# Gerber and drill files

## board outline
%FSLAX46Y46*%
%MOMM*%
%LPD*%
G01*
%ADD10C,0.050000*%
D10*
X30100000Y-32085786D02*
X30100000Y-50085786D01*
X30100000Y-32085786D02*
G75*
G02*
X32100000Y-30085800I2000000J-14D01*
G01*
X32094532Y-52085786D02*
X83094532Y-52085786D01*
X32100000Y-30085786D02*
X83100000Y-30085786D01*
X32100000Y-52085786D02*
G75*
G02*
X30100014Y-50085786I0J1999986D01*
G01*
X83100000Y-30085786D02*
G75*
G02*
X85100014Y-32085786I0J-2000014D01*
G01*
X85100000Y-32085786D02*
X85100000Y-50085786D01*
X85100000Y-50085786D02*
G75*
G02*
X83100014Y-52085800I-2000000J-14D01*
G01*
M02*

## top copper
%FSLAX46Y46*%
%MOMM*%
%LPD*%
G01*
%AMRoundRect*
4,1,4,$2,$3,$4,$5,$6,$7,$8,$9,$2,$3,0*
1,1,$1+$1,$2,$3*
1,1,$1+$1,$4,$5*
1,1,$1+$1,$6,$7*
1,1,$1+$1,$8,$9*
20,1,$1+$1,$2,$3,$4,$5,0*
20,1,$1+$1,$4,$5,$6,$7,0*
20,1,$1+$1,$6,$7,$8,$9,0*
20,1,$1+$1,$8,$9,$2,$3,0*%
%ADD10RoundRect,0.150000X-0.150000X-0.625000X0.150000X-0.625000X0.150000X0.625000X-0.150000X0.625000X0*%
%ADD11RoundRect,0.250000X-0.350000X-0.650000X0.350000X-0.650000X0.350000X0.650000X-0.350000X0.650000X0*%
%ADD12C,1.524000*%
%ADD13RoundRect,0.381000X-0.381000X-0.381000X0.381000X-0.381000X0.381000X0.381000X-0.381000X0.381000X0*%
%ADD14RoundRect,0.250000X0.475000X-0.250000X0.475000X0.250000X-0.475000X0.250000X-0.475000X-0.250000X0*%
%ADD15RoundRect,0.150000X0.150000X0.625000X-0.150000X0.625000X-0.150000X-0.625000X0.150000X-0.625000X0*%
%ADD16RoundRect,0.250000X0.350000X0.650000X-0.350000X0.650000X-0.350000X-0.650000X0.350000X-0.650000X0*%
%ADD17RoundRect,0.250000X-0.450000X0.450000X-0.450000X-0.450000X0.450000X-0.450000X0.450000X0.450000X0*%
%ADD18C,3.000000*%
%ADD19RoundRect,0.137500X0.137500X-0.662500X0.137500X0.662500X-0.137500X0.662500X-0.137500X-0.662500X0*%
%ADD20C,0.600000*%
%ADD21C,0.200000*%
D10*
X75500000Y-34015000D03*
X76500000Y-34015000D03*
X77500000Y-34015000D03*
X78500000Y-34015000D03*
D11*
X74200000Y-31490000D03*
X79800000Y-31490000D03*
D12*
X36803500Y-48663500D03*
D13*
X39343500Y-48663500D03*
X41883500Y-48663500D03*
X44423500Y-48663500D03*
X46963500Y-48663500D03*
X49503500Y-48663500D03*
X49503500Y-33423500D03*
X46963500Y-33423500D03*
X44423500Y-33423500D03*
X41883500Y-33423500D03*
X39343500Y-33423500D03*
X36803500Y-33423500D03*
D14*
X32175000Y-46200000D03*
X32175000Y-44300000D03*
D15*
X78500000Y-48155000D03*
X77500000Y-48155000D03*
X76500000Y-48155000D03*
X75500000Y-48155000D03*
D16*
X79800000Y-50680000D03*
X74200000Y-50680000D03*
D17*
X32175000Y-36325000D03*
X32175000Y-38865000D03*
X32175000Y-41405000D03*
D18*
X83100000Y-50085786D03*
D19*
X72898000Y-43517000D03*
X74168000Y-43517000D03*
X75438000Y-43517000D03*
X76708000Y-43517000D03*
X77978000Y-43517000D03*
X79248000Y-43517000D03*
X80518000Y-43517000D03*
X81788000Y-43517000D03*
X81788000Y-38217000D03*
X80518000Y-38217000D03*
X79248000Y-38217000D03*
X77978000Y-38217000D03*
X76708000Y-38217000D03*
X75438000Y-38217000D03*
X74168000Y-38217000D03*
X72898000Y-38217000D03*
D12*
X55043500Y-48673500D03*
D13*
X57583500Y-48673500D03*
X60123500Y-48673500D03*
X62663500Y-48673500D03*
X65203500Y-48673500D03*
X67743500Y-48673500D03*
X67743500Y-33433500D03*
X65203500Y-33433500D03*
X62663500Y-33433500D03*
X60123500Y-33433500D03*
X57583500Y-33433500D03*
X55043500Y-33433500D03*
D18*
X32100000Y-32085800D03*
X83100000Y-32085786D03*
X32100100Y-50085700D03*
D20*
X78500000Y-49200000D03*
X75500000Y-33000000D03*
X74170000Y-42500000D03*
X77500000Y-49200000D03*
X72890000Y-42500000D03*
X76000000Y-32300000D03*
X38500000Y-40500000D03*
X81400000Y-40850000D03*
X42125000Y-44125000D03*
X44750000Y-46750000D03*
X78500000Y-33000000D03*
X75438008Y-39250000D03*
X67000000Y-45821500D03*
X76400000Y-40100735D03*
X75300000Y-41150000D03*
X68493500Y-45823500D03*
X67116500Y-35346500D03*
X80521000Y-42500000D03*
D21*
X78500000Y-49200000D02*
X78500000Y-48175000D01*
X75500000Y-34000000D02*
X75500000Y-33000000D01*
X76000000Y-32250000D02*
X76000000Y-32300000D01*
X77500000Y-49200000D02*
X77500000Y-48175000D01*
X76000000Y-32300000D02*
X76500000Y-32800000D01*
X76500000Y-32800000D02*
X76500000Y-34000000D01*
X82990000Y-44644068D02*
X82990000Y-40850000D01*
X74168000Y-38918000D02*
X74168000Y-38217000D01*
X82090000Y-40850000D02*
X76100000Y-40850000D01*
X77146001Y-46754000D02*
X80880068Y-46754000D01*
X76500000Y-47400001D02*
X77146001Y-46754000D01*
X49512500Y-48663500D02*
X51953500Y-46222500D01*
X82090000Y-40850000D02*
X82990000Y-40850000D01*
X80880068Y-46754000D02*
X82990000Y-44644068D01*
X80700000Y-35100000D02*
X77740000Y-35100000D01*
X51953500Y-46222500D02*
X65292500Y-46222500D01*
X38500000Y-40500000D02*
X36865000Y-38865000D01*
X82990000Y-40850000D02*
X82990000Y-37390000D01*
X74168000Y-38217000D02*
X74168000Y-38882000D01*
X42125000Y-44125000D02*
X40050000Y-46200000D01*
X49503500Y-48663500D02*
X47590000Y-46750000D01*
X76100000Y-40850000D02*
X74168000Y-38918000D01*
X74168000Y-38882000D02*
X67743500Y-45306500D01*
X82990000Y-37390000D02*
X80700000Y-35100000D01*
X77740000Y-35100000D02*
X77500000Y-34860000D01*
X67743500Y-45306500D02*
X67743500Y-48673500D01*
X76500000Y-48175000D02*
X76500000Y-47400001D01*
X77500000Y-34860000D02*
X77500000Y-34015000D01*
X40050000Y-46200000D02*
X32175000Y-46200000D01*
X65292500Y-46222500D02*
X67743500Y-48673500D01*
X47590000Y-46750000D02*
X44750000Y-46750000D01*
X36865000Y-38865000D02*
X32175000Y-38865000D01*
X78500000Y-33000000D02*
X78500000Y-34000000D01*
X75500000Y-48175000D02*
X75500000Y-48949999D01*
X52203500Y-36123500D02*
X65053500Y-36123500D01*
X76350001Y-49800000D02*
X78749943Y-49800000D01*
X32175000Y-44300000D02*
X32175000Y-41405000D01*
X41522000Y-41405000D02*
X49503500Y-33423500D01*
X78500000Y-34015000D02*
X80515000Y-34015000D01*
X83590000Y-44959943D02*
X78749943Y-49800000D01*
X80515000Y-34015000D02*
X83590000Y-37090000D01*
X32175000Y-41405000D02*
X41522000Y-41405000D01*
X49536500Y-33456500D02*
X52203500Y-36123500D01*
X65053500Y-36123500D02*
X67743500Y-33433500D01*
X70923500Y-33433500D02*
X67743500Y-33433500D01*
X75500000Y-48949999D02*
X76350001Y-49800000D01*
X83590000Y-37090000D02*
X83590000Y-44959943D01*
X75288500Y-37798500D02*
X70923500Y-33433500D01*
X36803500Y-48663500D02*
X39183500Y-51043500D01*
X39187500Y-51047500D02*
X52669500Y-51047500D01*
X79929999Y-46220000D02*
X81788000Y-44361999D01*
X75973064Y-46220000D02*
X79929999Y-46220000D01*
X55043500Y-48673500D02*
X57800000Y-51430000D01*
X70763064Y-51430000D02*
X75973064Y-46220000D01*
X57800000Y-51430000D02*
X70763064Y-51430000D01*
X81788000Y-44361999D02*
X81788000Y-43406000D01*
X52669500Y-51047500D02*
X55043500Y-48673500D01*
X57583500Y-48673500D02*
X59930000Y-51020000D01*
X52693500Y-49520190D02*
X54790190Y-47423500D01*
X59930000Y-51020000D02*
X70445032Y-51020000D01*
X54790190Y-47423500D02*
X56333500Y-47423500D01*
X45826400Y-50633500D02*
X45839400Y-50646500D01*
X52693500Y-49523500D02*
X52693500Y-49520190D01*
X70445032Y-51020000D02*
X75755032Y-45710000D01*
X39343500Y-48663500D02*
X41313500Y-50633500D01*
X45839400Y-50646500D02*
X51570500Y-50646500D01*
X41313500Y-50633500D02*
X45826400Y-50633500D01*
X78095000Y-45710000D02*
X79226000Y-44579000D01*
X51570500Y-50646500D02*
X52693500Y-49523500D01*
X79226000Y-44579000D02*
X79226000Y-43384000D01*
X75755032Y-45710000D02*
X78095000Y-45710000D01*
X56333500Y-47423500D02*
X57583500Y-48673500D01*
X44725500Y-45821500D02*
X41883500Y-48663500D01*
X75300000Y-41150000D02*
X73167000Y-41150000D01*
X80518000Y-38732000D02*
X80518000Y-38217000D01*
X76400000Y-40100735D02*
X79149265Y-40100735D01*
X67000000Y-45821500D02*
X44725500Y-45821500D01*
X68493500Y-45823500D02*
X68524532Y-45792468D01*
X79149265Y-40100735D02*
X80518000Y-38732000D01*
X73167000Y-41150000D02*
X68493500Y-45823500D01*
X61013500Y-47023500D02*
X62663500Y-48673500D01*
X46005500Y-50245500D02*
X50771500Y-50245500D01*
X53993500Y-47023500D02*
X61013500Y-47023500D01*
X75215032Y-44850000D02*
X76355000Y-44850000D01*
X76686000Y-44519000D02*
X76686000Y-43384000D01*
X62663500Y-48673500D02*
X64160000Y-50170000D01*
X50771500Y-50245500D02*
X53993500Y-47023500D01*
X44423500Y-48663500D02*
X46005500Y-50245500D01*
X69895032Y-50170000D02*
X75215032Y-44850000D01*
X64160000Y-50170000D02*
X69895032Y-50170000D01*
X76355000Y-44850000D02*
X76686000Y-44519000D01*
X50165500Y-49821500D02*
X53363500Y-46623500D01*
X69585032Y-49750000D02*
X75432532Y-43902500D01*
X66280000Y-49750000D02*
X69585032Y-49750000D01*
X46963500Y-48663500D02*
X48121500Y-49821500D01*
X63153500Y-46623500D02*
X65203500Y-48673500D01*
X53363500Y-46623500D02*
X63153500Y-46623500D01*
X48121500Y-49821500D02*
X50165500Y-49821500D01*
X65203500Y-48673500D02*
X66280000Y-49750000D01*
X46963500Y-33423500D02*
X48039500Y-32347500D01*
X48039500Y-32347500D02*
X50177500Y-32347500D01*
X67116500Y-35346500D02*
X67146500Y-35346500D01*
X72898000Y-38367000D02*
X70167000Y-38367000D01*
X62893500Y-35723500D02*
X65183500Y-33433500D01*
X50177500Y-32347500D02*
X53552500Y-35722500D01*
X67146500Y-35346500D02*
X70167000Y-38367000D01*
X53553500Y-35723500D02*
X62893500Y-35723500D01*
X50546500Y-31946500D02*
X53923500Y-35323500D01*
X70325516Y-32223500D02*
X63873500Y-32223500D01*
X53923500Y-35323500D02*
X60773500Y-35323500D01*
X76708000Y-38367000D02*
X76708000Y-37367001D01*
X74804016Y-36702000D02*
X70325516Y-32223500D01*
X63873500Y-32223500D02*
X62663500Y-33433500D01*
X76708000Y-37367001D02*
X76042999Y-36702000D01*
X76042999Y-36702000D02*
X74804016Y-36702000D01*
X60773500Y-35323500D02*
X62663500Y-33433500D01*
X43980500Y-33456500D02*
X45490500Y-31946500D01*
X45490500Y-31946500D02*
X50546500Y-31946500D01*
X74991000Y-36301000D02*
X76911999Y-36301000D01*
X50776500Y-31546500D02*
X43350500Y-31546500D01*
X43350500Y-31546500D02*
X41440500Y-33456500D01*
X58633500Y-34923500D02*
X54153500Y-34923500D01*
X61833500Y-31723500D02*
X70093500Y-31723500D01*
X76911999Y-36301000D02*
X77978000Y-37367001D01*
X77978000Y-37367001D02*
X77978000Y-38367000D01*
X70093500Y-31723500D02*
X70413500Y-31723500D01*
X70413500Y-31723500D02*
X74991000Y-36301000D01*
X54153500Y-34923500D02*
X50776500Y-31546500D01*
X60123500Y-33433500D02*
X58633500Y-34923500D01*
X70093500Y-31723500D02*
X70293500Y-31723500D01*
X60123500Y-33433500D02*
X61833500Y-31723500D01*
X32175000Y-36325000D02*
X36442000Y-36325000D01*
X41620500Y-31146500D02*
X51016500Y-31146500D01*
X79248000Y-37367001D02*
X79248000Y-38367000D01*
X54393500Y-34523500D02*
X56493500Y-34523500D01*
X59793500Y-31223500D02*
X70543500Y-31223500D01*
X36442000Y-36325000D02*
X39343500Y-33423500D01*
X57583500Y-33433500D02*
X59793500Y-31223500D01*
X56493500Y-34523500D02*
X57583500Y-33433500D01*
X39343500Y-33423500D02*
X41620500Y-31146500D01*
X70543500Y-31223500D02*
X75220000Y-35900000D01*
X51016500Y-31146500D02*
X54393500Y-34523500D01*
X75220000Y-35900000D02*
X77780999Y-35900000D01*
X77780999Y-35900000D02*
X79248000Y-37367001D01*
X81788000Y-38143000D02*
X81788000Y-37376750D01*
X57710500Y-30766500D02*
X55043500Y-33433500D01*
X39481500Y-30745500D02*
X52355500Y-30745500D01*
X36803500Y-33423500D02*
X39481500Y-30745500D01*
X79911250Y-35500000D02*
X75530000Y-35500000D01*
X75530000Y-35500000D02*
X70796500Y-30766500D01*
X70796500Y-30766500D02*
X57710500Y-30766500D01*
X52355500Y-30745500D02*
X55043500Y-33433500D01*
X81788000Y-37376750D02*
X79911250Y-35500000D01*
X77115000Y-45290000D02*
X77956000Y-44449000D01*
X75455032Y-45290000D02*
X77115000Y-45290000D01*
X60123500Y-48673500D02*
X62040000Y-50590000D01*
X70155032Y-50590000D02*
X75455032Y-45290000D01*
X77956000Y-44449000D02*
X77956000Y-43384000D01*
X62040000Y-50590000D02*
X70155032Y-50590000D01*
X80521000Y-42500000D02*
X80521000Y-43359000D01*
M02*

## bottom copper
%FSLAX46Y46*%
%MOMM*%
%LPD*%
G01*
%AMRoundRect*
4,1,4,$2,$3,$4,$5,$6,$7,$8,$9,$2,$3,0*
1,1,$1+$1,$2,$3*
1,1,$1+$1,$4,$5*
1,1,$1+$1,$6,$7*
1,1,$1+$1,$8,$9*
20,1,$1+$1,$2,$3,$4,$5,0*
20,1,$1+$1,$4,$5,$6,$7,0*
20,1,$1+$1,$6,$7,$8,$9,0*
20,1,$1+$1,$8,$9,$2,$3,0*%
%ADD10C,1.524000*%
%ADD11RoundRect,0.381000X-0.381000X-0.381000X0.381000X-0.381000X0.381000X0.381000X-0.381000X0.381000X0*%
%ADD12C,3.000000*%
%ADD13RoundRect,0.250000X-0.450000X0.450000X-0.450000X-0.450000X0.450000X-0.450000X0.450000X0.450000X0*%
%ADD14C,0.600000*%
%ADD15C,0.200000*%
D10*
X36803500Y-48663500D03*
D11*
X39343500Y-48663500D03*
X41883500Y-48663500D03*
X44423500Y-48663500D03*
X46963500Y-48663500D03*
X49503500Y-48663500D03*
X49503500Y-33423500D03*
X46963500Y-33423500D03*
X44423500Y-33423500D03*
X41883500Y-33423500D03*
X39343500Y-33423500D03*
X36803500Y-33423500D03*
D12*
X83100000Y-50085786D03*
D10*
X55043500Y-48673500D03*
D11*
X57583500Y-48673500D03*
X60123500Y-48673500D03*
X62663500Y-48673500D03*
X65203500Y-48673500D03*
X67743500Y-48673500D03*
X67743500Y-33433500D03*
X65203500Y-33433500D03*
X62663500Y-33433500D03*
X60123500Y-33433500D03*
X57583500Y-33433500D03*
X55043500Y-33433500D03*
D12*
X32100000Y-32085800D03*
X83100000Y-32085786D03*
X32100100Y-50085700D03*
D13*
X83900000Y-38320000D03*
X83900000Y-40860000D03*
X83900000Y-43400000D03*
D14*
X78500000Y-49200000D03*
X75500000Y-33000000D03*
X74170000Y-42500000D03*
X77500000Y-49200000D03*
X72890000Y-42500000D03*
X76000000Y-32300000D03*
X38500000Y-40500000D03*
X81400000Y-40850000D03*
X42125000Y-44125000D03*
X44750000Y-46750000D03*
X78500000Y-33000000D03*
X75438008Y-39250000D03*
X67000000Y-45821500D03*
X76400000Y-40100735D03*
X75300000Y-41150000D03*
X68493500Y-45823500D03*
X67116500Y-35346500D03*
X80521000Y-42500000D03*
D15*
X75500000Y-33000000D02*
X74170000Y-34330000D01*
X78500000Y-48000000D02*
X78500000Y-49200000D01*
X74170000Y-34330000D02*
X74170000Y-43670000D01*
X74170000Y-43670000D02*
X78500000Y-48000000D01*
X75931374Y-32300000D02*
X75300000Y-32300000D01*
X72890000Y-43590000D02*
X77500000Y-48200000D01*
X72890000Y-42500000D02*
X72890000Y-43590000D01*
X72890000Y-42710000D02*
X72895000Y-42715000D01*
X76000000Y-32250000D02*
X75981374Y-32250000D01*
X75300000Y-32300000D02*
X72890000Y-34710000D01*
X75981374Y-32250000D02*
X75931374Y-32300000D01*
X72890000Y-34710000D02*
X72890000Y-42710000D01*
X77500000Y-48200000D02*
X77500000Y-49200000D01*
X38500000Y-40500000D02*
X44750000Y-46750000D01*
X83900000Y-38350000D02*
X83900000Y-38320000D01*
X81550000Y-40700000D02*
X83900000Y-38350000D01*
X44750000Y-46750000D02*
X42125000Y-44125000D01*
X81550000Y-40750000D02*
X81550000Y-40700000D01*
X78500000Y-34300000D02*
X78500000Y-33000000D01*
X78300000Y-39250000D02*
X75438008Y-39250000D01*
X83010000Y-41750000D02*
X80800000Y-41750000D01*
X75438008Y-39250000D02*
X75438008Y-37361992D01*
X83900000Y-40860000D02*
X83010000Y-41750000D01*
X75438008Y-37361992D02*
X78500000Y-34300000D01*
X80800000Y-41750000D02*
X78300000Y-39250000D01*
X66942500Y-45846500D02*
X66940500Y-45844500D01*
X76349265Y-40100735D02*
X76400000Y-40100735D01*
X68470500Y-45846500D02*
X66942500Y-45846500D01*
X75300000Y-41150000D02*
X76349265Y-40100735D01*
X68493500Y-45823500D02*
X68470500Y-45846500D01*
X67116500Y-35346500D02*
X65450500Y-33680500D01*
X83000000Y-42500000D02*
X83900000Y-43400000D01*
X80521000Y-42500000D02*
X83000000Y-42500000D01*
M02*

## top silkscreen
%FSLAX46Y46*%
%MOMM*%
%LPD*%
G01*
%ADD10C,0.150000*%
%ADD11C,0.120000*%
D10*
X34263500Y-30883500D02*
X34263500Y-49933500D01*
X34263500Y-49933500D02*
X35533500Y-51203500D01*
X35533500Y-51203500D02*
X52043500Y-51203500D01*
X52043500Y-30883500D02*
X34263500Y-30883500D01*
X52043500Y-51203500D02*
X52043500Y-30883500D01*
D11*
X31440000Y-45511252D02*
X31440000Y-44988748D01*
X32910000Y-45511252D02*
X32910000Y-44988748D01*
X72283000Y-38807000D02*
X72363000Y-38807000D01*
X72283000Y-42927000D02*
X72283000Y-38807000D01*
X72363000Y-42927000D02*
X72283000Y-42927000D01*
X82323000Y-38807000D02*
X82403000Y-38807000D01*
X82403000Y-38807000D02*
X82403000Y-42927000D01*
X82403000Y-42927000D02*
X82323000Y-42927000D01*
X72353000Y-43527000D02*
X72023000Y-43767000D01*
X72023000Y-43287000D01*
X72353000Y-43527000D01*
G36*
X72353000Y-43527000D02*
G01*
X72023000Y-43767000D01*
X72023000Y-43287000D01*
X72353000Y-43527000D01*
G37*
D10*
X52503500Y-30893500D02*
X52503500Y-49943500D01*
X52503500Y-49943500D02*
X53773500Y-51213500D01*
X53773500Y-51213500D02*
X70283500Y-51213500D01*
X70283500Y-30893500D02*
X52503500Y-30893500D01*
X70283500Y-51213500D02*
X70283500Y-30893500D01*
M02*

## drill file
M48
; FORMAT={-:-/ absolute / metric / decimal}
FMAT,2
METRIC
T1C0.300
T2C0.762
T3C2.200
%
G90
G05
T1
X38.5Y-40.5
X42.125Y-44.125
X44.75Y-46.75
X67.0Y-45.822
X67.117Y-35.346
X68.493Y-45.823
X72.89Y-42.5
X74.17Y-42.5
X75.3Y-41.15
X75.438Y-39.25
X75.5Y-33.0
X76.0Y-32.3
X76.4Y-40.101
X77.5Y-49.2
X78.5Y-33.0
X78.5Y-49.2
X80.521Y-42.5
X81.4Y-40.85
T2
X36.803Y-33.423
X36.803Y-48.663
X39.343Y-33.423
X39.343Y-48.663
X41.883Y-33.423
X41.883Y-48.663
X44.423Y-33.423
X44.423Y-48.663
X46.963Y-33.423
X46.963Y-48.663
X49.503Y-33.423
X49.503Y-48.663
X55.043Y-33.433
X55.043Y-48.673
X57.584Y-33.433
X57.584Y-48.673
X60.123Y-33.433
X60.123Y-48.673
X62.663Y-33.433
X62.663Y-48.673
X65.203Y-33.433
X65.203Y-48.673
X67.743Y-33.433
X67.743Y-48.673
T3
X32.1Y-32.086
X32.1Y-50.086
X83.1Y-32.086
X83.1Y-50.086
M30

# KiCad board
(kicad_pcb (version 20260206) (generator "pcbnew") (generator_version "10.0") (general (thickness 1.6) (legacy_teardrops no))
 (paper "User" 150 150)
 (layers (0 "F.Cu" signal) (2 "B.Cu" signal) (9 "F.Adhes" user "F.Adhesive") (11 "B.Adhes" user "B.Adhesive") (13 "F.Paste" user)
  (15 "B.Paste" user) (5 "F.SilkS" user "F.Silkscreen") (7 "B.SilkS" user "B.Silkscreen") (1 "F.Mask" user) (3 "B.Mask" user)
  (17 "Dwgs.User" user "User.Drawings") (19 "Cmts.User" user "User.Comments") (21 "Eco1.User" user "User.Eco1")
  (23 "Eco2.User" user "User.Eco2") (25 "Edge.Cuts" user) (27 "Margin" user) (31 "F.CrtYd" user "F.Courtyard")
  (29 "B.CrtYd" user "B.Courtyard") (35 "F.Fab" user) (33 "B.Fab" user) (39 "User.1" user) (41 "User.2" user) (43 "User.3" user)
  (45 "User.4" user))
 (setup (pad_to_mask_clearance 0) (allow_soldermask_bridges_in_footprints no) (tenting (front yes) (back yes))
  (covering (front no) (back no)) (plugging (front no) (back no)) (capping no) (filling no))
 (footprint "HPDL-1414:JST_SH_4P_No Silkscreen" (layer "F.Cu") (at 77 32.69)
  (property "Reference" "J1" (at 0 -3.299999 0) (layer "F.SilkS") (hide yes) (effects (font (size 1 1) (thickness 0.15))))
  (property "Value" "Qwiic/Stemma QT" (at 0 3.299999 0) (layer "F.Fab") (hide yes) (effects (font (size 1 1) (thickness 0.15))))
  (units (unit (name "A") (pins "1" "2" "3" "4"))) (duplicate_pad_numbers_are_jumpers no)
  (pad "1" smd roundrect (at -1.5 1.325) (size 0.6 1.55) (layers "F.Cu" "F.Mask" "F.Paste") (roundrect_rratio 0.25) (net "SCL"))
  (pad "2" smd roundrect (at -0.5 1.325) (size 0.6 1.55) (layers "F.Cu" "F.Mask" "F.Paste") (roundrect_rratio 0.25) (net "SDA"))
  (pad "3" smd roundrect (at 0.5 1.325) (size 0.6 1.55) (layers "F.Cu" "F.Mask" "F.Paste") (roundrect_rratio 0.25) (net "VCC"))
  (pad "4" smd roundrect (at 1.5 1.325) (size 0.6 1.55) (layers "F.Cu" "F.Mask" "F.Paste") (roundrect_rratio 0.25) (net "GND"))
  (pad "MP" smd roundrect (at -2.8 -1.2) (size 1.2 1.8) (layers "F.Cu" "F.Mask" "F.Paste") (roundrect_rratio 0.208333))
  (pad "MP" smd roundrect (at 2.8 -1.2) (size 1.2 1.8) (layers "F.Cu" "F.Mask" "F.Paste") (roundrect_rratio 0.208333)))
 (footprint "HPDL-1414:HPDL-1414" (layer "F.Cu") (at 43.1535 41.0435)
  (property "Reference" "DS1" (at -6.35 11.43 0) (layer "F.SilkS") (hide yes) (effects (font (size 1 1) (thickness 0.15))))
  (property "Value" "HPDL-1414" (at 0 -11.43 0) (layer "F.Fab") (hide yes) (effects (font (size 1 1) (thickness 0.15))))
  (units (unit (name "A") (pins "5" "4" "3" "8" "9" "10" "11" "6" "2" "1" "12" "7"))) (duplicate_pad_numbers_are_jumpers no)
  (fp_line (start -8.89 -10.16) (end -8.89 8.89) (stroke (width 0.15) (type solid)) (layer "F.SilkS"))
  (fp_line (start -8.89 8.89) (end -7.62 10.16) (stroke (width 0.15) (type solid)) (layer "F.SilkS"))
  (fp_line (start -7.62 10.16) (end 8.89 10.16) (stroke (width 0.15) (type solid)) (layer "F.SilkS"))
  (fp_line (start 8.89 -10.16) (end -8.89 -10.16) (stroke (width 0.15) (type solid)) (layer "F.SilkS"))
  (fp_line (start 8.89 10.16) (end 8.89 -10.16) (stroke (width 0.15) (type solid)) (layer "F.SilkS"))
  (pad "1" thru_hole circle (at -6.35 7.62) (size 1.524 1.524) (drill 0.762) (layers "*.Cu" "*.Mask") (remove_unused_layers no) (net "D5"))
  (pad "2" thru_hole roundrect (at -3.81 7.62) (size 1.524 1.524) (drill 0.762) (layers "*.Cu" "*.Mask") (remove_unused_layers no)
   (roundrect_rratio 0.25) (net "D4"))
  (pad "3" thru_hole roundrect (at -1.27 7.62) (size 1.524 1.524) (drill 0.762) (layers "*.Cu" "*.Mask") (remove_unused_layers no)
   (roundrect_rratio 0.25) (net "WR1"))
  (pad "4" thru_hole roundrect (at 1.27 7.62) (size 1.524 1.524) (drill 0.762) (layers "*.Cu" "*.Mask") (remove_unused_layers no)
   (roundrect_rratio 0.25) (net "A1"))
  (pad "5" thru_hole roundrect (at 3.81 7.62) (size 1.524 1.524) (drill 0.762) (layers "*.Cu" "*.Mask") (remove_unused_layers no)
   (roundrect_rratio 0.25) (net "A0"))
  (pad "6" thru_hole roundrect (at 6.35 7.62) (size 1.524 1.524) (drill 0.762) (layers "*.Cu" "*.Mask") (remove_unused_layers no)
   (roundrect_rratio 0.25) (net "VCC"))
  (pad "7" thru_hole roundrect (at 6.35 -7.62) (size 1.524 1.524) (drill 0.762) (layers "*.Cu" "*.Mask") (remove_unused_layers no)
   (roundrect_rratio 0.25) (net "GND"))
  (pad "8" thru_hole roundrect (at 3.81 -7.62) (size 1.524 1.524) (drill 0.762) (layers "*.Cu" "*.Mask") (remove_unused_layers no)
   (roundrect_rratio 0.25) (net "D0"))
  (pad "9" thru_hole roundrect (at 1.27 -7.62) (size 1.524 1.524) (drill 0.762) (layers "*.Cu" "*.Mask") (remove_unused_layers no)
   (roundrect_rratio 0.25) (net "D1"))
  (pad "10" thru_hole roundrect (at -1.27 -7.62) (size 1.524 1.524) (drill 0.762) (layers "*.Cu" "*.Mask") (remove_unused_layers no)
   (roundrect_rratio 0.25) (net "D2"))
  (pad "11" thru_hole roundrect (at -3.81 -7.62) (size 1.524 1.524) (drill 0.762) (layers "*.Cu" "*.Mask") (remove_unused_layers no)
   (roundrect_rratio 0.25) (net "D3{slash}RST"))
  (pad "12" thru_hole roundrect (at -6.35 -7.62) (size 1.524 1.524) (drill 0.762) (layers "*.Cu" "*.Mask") (remove_unused_layers no)
   (roundrect_rratio 0.25) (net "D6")))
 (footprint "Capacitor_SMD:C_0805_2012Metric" (layer "F.Cu") (at 32.175 45.25 90)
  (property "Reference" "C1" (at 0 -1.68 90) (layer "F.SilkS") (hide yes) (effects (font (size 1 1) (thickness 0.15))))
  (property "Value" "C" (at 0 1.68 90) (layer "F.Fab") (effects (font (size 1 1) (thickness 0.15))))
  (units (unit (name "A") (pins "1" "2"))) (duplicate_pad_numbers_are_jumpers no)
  (fp_line (start -0.261252 -0.735) (end 0.261252 -0.735) (stroke (width 0.12) (type solid)) (layer "F.SilkS"))
  (fp_line (start -0.261252 0.735) (end 0.261252 0.735) (stroke (width 0.12) (type solid)) (layer "F.SilkS"))
  (pad "1" smd roundrect (at -0.95 0 90) (size 1 1.45) (layers "F.Cu" "F.Mask" "F.Paste") (roundrect_rratio 0.25) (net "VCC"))
  (pad "2" smd roundrect (at 0.95 0 90) (size 1 1.45) (layers "F.Cu" "F.Mask" "F.Paste") (roundrect_rratio 0.25) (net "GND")))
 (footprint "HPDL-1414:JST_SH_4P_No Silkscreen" (layer "F.Cu") (at 77 49.48 180)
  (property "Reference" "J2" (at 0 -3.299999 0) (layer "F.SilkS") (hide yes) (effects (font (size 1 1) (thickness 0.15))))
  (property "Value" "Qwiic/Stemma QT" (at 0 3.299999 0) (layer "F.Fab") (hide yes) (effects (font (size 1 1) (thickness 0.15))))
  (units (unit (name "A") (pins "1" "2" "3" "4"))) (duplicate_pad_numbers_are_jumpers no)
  (pad "1" smd roundrect (at -1.5 1.325 180) (size 0.6 1.55) (layers "F.Cu" "F.Mask" "F.Paste") (roundrect_rratio 0.25) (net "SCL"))
  (pad "2" smd roundrect (at -0.5 1.325 180) (size 0.6 1.55) (layers "F.Cu" "F.Mask" "F.Paste") (roundrect_rratio 0.25) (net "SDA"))
  (pad "3" smd roundrect (at 0.5 1.325 180) (size 0.6 1.55) (layers "F.Cu" "F.Mask" "F.Paste") (roundrect_rratio 0.25) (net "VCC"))
  (pad "4" smd roundrect (at 1.5 1.325 180) (size 0.6 1.55) (layers "F.Cu" "F.Mask" "F.Paste") (roundrect_rratio 0.25) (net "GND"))
  (pad "MP" smd roundrect (at -2.8 -1.2 180) (size 1.2 1.8) (layers "F.Cu" "F.Mask" "F.Paste") (roundrect_rratio 0.208333))
  (pad "MP" smd roundrect (at 2.8 -1.2 180) (size 1.2 1.8) (layers "F.Cu" "F.Mask" "F.Paste") (roundrect_rratio 0.208333)))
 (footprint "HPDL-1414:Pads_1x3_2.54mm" (layer "F.Cu") (at 32.175 36.325 -90)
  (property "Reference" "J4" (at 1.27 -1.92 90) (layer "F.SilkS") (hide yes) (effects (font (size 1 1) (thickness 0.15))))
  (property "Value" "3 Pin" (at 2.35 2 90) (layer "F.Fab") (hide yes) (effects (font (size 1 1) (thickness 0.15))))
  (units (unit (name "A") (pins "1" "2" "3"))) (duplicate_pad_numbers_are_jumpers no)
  (pad "1" smd roundrect (at 0 0 270) (size 1.4 1.4) (layers "F.Cu" "F.Mask") (roundrect_rratio 0.1785714286) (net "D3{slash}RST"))
  (pad "2" smd roundrect (at 2.54 0 270) (size 1.4 1.4) (layers "F.Cu" "F.Mask") (roundrect_rratio 0.1785714286) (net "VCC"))
  (pad "3" smd roundrect (at 5.08 0 270) (size 1.4 1.4) (layers "F.Cu" "F.Mask") (roundrect_rratio 0.1785714286) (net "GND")))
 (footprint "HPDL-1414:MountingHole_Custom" (layer "F.Cu") (at 83.1 50.085786)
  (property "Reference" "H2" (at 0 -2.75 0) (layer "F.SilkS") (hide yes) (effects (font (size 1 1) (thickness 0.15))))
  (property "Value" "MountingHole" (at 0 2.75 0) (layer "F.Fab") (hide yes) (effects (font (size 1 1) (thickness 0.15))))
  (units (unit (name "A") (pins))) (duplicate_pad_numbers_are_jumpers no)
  (pad "1" thru_hole circle (at 0 0) (size 3 3) (drill 2.2) (layers "*.Cu" "*.Mask") (remove_unused_layers no)))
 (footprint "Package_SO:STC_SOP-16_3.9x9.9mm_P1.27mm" (layer "F.Cu") (at 77.343 40.867 90)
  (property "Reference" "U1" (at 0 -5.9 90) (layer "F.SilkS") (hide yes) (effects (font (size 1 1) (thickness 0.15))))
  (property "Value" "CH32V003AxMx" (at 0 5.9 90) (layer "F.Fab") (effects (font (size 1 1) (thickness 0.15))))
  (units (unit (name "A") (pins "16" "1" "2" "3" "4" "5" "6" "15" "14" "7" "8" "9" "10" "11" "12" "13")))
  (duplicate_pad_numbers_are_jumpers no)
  (fp_line (start 2.06 -5.06) (end 2.06 -4.98) (stroke (width 0.12) (type solid)) (layer "F.SilkS"))
  (fp_line (start -2.06 -5.06) (end 2.06 -5.06) (stroke (width 0.12) (type solid)) (layer "F.SilkS"))
  (fp_line (start -2.06 -4.98) (end -2.06 -5.06) (stroke (width 0.12) (type solid)) (layer "F.SilkS"))
  (fp_line (start 2.06 4.98) (end 2.06 5.06) (stroke (width 0.12) (type solid)) (layer "F.SilkS"))
  (fp_line (start 2.06 5.06) (end -2.06 5.06) (stroke (width 0.12) (type solid)) (layer "F.SilkS"))
  (fp_line (start -2.06 5.06) (end -2.06 4.98) (stroke (width 0.12) (type solid)) (layer "F.SilkS"))
  (fp_poly (pts (xy -2.66 -4.99) (xy -2.9 -5.32) (xy -2.42 -5.32)) (stroke (width 0.12) (type solid)) (fill yes) (layer "F.SilkS"))
  (pad "1" smd roundrect (at -2.65 -4.445 90) (size 1.6 0.55) (layers "F.Cu" "F.Mask" "F.Paste") (roundrect_rratio 0.25) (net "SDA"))
  (pad "2" smd roundrect (at -2.65 -3.175 90) (size 1.6 0.55) (layers "F.Cu" "F.Mask" "F.Paste") (roundrect_rratio 0.25) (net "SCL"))
  (pad "3" smd roundrect (at -2.65 -1.905 90) (size 1.6 0.55) (layers "F.Cu" "F.Mask" "F.Paste") (roundrect_rratio 0.25) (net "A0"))
  (pad "4" smd roundrect (at -2.65 -0.635 90) (size 1.6 0.55) (layers "F.Cu" "F.Mask" "F.Paste") (roundrect_rratio 0.25) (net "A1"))
  (pad "5" smd roundrect (at -2.65 0.635 90) (size 1.6 0.55) (layers "F.Cu" "F.Mask" "F.Paste") (roundrect_rratio 0.25) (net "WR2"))
  (pad "6" smd roundrect (at -2.65 1.905 90) (size 1.6 0.55) (layers "F.Cu" "F.Mask" "F.Paste") (roundrect_rratio 0.25) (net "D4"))
  (pad "7" smd roundrect (at -2.65 3.175 90) (size 1.6 0.55) (layers "F.Cu" "F.Mask" "F.Paste") (roundrect_rratio 0.25) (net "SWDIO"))
  (pad "8" smd roundrect (at -2.65 4.445 90) (size 1.6 0.55) (layers "F.Cu" "F.Mask" "F.Paste") (roundrect_rratio 0.25) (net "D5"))
  (pad "9" smd roundrect (at 2.65 4.445 90) (size 1.6 0.55) (layers "F.Cu" "F.Mask" "F.Paste") (roundrect_rratio 0.25) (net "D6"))
  (pad "10" smd roundrect (at 2.65 3.175 90) (size 1.6 0.55) (layers "F.Cu" "F.Mask" "F.Paste") (roundrect_rratio 0.25) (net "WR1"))
  (pad "11" smd roundrect (at 2.65 1.905 90) (size 1.6 0.55) (layers "F.Cu" "F.Mask" "F.Paste") (roundrect_rratio 0.25) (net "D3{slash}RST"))
  (pad "12" smd roundrect (at 2.65 0.635 90) (size 1.6 0.55) (layers "F.Cu" "F.Mask" "F.Paste") (roundrect_rratio 0.25) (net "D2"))
  (pad "13" smd roundrect (at 2.65 -0.635 90) (size 1.6 0.55) (layers "F.Cu" "F.Mask" "F.Paste") (roundrect_rratio 0.25) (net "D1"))
  (pad "14" smd roundrect (at 2.65 -1.905 90) (size 1.6 0.55) (layers "F.Cu" "F.Mask" "F.Paste") (roundrect_rratio 0.25) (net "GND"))
  (pad "15" smd roundrect (at 2.65 -3.175 90) (size 1.6 0.55) (layers "F.Cu" "F.Mask" "F.Paste") (roundrect_rratio 0.25) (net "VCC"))
  (pad "16" smd roundrect (at 2.65 -4.445 90) (size 1.6 0.55) (layers "F.Cu" "F.Mask" "F.Paste") (roundrect_rratio 0.25) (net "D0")))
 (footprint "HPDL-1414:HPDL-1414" (layer "F.Cu") (at 61.3935 41.0535)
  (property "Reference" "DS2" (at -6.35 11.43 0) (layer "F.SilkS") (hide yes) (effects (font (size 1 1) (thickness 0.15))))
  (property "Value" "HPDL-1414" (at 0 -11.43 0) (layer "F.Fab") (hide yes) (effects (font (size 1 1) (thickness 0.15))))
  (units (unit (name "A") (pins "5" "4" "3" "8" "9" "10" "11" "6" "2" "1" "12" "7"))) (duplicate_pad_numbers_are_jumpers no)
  (fp_line (start -8.89 -10.16) (end -8.89 8.89) (stroke (width 0.15) (type solid)) (layer "F.SilkS"))
  (fp_line (start -8.89 8.89) (end -7.62 10.16) (stroke (width 0.15) (type solid)) (layer "F.SilkS"))
  (fp_line (start -7.62 10.16) (end 8.89 10.16) (stroke (width 0.15) (type solid)) (layer "F.SilkS"))
  (fp_line (start 8.89 -10.16) (end -8.89 -10.16) (stroke (width 0.15) (type solid)) (layer "F.SilkS"))
  (fp_line (start 8.89 10.16) (end 8.89 -10.16) (stroke (width 0.15) (type solid)) (layer "F.SilkS"))
  (pad "1" thru_hole circle (at -6.35 7.62) (size 1.524 1.524) (drill 0.762) (layers "*.Cu" "*.Mask") (remove_unused_layers no) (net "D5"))
  (pad "2" thru_hole roundrect (at -3.81 7.62) (size 1.524 1.524) (drill 0.762) (layers "*.Cu" "*.Mask") (remove_unused_layers no)
   (roundrect_rratio 0.25) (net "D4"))
  (pad "3" thru_hole roundrect (at -1.27 7.62) (size 1.524 1.524) (drill 0.762) (layers "*.Cu" "*.Mask") (remove_unused_layers no)
   (roundrect_rratio 0.25) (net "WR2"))
  (pad "4" thru_hole roundrect (at 1.27 7.62) (size 1.524 1.524) (drill 0.762) (layers "*.Cu" "*.Mask") (remove_unused_layers no)
   (roundrect_rratio 0.25) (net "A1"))
  (pad "5" thru_hole roundrect (at 3.81 7.62) (size 1.524 1.524) (drill 0.762) (layers "*.Cu" "*.Mask") (remove_unused_layers no)
   (roundrect_rratio 0.25) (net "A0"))
  (pad "6" thru_hole roundrect (at 6.35 7.62) (size 1.524 1.524) (drill 0.762) (layers "*.Cu" "*.Mask") (remove_unused_layers no)
   (roundrect_rratio 0.25) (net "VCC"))
  (pad "7" thru_hole roundrect (at 6.35 -7.62) (size 1.524 1.524) (drill 0.762) (layers "*.Cu" "*.Mask") (remove_unused_layers no)
   (roundrect_rratio 0.25) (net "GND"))
  (pad "8" thru_hole roundrect (at 3.81 -7.62) (size 1.524 1.524) (drill 0.762) (layers "*.Cu" "*.Mask") (remove_unused_layers no)
   (roundrect_rratio 0.25) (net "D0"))
  (pad "9" thru_hole roundrect (at 1.27 -7.62) (size 1.524 1.524) (drill 0.762) (layers "*.Cu" "*.Mask") (remove_unused_layers no)
   (roundrect_rratio 0.25) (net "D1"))
  (pad "10" thru_hole roundrect (at -1.27 -7.62) (size 1.524 1.524) (drill 0.762) (layers "*.Cu" "*.Mask") (remove_unused_layers no)
   (roundrect_rratio 0.25) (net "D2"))
  (pad "11" thru_hole roundrect (at -3.81 -7.62) (size 1.524 1.524) (drill 0.762) (layers "*.Cu" "*.Mask") (remove_unused_layers no)
   (roundrect_rratio 0.25) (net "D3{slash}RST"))
  (pad "12" thru_hole roundrect (at -6.35 -7.62) (size 1.524 1.524) (drill 0.762) (layers "*.Cu" "*.Mask") (remove_unused_layers no)
   (roundrect_rratio 0.25) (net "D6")))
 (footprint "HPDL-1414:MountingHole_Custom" (layer "F.Cu") (at 32.1 32.0858)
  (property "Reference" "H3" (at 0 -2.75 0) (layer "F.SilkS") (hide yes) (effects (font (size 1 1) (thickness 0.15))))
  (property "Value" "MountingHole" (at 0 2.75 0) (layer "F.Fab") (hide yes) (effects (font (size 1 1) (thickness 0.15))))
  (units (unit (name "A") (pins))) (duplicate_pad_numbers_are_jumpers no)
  (pad "1" thru_hole circle (at 0 0) (size 3 3) (drill 2.2) (layers "*.Cu" "*.Mask") (remove_unused_layers no)))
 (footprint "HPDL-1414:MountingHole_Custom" (layer "F.Cu") (at 83.1 32.085786)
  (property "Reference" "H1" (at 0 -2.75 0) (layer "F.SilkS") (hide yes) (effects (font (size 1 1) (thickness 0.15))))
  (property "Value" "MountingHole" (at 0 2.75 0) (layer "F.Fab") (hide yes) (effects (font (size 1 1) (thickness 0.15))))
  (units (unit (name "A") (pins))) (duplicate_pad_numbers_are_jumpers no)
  (pad "1" thru_hole circle (at 0 0) (size 3 3) (drill 2.2) (layers "*.Cu" "*.Mask") (remove_unused_layers no)))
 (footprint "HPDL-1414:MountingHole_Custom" (layer "F.Cu") (at 32.1001 50.0857)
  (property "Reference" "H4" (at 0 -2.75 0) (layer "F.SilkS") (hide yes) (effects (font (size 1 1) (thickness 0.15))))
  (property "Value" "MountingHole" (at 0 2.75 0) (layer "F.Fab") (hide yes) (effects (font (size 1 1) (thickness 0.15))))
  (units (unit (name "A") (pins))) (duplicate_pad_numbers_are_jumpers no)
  (pad "1" thru_hole circle (at 0 0) (size 3 3) (drill 2.2) (layers "*.Cu" "*.Mask") (remove_unused_layers no)))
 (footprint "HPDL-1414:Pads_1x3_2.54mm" (layer "B.Cu") (at 83.9 38.32 -90)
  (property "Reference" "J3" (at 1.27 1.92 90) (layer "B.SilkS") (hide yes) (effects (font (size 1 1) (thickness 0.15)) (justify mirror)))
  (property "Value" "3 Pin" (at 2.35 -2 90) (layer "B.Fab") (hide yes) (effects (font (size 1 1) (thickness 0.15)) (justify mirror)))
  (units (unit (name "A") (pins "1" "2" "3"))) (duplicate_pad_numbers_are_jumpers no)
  (pad "1" smd roundrect (at 0 0 270) (size 1.4 1.4) (layers "B.Cu" "B.Mask") (roundrect_rratio 0.1785714286) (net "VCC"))
  (pad "2" smd roundrect (at 2.54 0 270) (size 1.4 1.4) (layers "B.Cu" "B.Mask") (roundrect_rratio 0.1785714286) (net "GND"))
  (pad "3" smd roundrect (at 5.08 0 270) (size 1.4 1.4) (layers "B.Cu" "B.Mask") (roundrect_rratio 0.1785714286) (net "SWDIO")))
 (gr_line (start 30.1 32.085786) (end 30.1 50.085786) (stroke (width 0.05) (type default)) (layer "Edge.Cuts"))
 (gr_arc (start 30.1 32.085786) (mid 30.685786 30.671572) (end 32.1 30.085786) (stroke (width 0.05) (type default)) (layer "Edge.Cuts"))
 (gr_line (start 32.094532 52.085786) (end 83.094532 52.085786) (stroke (width 0.05) (type default)) (layer "Edge.Cuts"))
 (gr_line (start 32.1 30.085786) (end 83.1 30.085786) (stroke (width 0.05) (type solid)) (layer "Edge.Cuts"))
 (gr_arc (start 32.1 52.085786) (mid 30.685786 51.5) (end 30.1 50.085786) (stroke (width 0.05) (type default)) (layer "Edge.Cuts"))
 (gr_arc (start 83.1 30.085786) (mid 84.514214 30.671572) (end 85.1 32.085786) (stroke (width 0.05) (type default)) (layer "Edge.Cuts"))
 (gr_line (start 85.1 32.085786) (end 85.1 50.085786) (stroke (width 0.05) (type default)) (layer "Edge.Cuts"))
 (gr_arc (start 85.1 50.085786) (mid 84.514223 51.500004) (end 83.100014 52.0858) (stroke (width 0.05) (type solid)) (layer "Edge.Cuts"))
 (segment (start 78.5 49.2) (end 78.5 48.175) (width 0.2) (layer "F.Cu") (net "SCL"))
 (segment (start 75.5 34) (end 75.5 33) (width 0.2) (layer "F.Cu") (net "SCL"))
 (via (at 78.5 49.2) (size 0.6) (drill 0.3) (layers "F.Cu" "B.Cu") (capping no) (covering (front no) (back no))
  (plugging (front no) (back no)) (filling no) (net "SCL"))
 (via (at 75.5 33) (size 0.6) (drill 0.3) (layers "F.Cu" "B.Cu") (capping no) (covering (front no) (back no))
  (plugging (front no) (back no)) (filling no) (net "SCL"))
 (via (at 74.17 42.5) (size 0.6) (drill 0.3) (layers "F.Cu" "B.Cu") (capping no) (covering (front no) (back no))
  (plugging (front no) (back no)) (filling no) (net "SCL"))
 (segment (start 75.5 33) (end 74.17 34.33) (width 0.2) (layer "B.Cu") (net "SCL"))
 (segment (start 78.5 48) (end 78.5 49.2) (width 0.2) (layer "B.Cu") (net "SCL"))
 (segment (start 74.17 34.33) (end 74.17 43.67) (width 0.2) (layer "B.Cu") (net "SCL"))
 (segment (start 74.17 43.67) (end 78.5 48) (width 0.2) (layer "B.Cu") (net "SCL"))
 (segment (start 76 32.25) (end 76 32.3) (width 0.2) (layer "F.Cu") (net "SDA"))
 (segment (start 77.5 49.2) (end 77.5 48.175) (width 0.2) (layer "F.Cu") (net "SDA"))
 (segment (start 76 32.3) (end 76.5 32.8) (width 0.2) (layer "F.Cu") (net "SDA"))
 (segment (start 76.5 32.8) (end 76.5 34) (width 0.2) (layer "F.Cu") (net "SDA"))
 (via (at 77.5 49.2) (size 0.6) (drill 0.3) (layers "F.Cu" "B.Cu") (capping no) (covering (front no) (back no))
  (plugging (front no) (back no)) (filling no) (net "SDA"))
 (via (at 72.89 42.5) (size 0.6) (drill 0.3) (layers "F.Cu" "B.Cu") (capping no) (covering (front no) (back no))
  (plugging (front no) (back no)) (filling no) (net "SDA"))
 (via (at 76 32.3) (size 0.6) (drill 0.3) (layers "F.Cu" "B.Cu") (capping no) (covering (front no) (back no))
  (plugging (front no) (back no)) (filling no) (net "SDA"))
 (segment (start 75.931374 32.3) (end 75.3 32.3) (width 0.2) (layer "B.Cu") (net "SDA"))
 (segment (start 72.89 43.59) (end 77.5 48.2) (width 0.2) (layer "B.Cu") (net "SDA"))
 (segment (start 72.89 42.5) (end 72.89 43.59) (width 0.2) (layer "B.Cu") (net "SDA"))
 (segment (start 72.89 42.71) (end 72.895 42.715) (width 0.2) (layer "B.Cu") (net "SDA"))
 (segment (start 76 32.25) (end 75.981374 32.25) (width 0.2) (layer "B.Cu") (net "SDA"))
 (segment (start 75.3 32.3) (end 72.89 34.71) (width 0.2) (layer "B.Cu") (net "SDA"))
 (segment (start 75.981374 32.25) (end 75.931374 32.3) (width 0.2) (layer "B.Cu") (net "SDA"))
 (segment (start 72.89 34.71) (end 72.89 42.71) (width 0.2) (layer "B.Cu") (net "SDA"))
 (segment (start 77.5 48.2) (end 77.5 49.2) (width 0.2) (layer "B.Cu") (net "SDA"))
 (segment (start 82.99 44.644068) (end 82.99 40.85) (width 0.2) (layer "F.Cu") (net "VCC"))
 (segment (start 74.168 38.918) (end 74.168 38.217) (width 0.2) (layer "F.Cu") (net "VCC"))
 (segment (start 82.09 40.85) (end 76.1 40.85) (width 0.2) (layer "F.Cu") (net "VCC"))
 (segment (start 77.146001 46.754) (end 80.880068 46.754) (width 0.2) (layer "F.Cu") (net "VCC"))
 (segment (start 76.5 47.400001) (end 77.146001 46.754) (width 0.2) (layer "F.Cu") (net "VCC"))
 (segment (start 49.5125 48.6635) (end 51.9535 46.2225) (width 0.2) (layer "F.Cu") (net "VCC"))
 (segment (start 82.09 40.85) (end 82.99 40.85) (width 0.2) (layer "F.Cu") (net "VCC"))
 (segment (start 80.880068 46.754) (end 82.99 44.644068) (width 0.2) (layer "F.Cu") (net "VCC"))
 (segment (start 80.7 35.1) (end 77.74 35.1) (width 0.2) (layer "F.Cu") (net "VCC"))
 (segment (start 51.9535 46.2225) (end 65.2925 46.2225) (width 0.2) (layer "F.Cu") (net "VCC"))
 (segment (start 38.5 40.5) (end 36.865 38.865) (width 0.2) (layer "F.Cu") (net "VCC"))
 (segment (start 82.99 40.85) (end 82.99 37.39) (width 0.2) (layer "F.Cu") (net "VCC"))
 (segment (start 74.168 38.217) (end 74.168 38.882) (width 0.2) (layer "F.Cu") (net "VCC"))
 (segment (start 42.125 44.125) (end 40.05 46.2) (width 0.2) (layer "F.Cu") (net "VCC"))
 (segment (start 49.5035 48.6635) (end 47.59 46.75) (width 0.2) (layer "F.Cu") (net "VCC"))
 (segment (start 76.1 40.85) (end 74.168 38.918) (width 0.2) (layer "F.Cu") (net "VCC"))
 (segment (start 74.168 38.882) (end 67.7435 45.3065) (width 0.2) (layer "F.Cu") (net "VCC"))
 (segment (start 82.99 37.39) (end 80.7 35.1) (width 0.2) (layer "F.Cu") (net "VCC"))
 (segment (start 77.74 35.1) (end 77.5 34.86) (width 0.2) (layer "F.Cu") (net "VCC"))
 (segment (start 67.7435 45.3065) (end 67.7435 48.6735) (width 0.2) (layer "F.Cu") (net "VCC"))
 (segment (start 76.5 48.175) (end 76.5 47.400001) (width 0.2) (layer "F.Cu") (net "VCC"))
 (segment (start 77.5 34.86) (end 77.5 34.015) (width 0.2) (layer "F.Cu") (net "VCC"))
 (segment (start 40.05 46.2) (end 32.175 46.2) (width 0.2) (layer "F.Cu") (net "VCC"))
 (segment (start 65.2925 46.2225) (end 67.7435 48.6735) (width 0.2) (layer "F.Cu") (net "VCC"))
 (segment (start 47.59 46.75) (end 44.75 46.75) (width 0.2) (layer "F.Cu") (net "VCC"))
 (segment (start 36.865 38.865) (end 32.175 38.865) (width 0.2) (layer "F.Cu") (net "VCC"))
 (via (at 38.5 40.5) (size 0.6) (drill 0.3) (layers "F.Cu" "B.Cu") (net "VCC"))
 (via (at 81.4 40.85) (size 0.6) (drill 0.3) (layers "F.Cu" "B.Cu") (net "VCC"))
 (via (at 42.125 44.125) (size 0.6) (drill 0.3) (layers "F.Cu" "B.Cu") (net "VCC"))
 (via (at 44.75 46.75) (size 0.6) (drill 0.3) (layers "F.Cu" "B.Cu") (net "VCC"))
 (segment (start 38.5 40.5) (end 44.75 46.75) (width 0.2) (layer "B.Cu") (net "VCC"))
 (segment (start 83.9 38.35) (end 83.9 38.32) (width 0.2) (layer "B.Cu") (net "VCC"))
 (segment (start 81.55 40.7) (end 83.9 38.35) (width 0.2) (layer "B.Cu") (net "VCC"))
 (segment (start 44.75 46.75) (end 42.125 44.125) (width 0.2) (layer "B.Cu") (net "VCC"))
 (segment (start 81.55 40.75) (end 81.55 40.7) (width 0.2) (layer "B.Cu") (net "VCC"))
 (segment (start 78.5 33) (end 78.5 34) (width 0.2) (layer "F.Cu") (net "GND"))
 (segment (start 75.5 48.175) (end 75.5 48.949999) (width 0.2) (layer "F.Cu") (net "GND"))
 (segment (start 52.2035 36.1235) (end 65.0535 36.1235) (width 0.2) (layer "F.Cu") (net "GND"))
 (segment (start 76.350001 49.8) (end 78.749943 49.8) (width 0.2) (layer "F.Cu") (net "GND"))
 (segment (start 32.175 44.3) (end 32.175 41.405) (width 0.2) (layer "F.Cu") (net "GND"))
 (segment (start 41.522 41.405) (end 49.5035 33.4235) (width 0.2) (layer "F.Cu") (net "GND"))
 (segment (start 78.5 34.015) (end 80.515 34.015) (width 0.2) (layer "F.Cu") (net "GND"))
 (segment (start 83.59 44.959943) (end 78.749943 49.8) (width 0.2) (layer "F.Cu") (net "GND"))
 (segment (start 80.515 34.015) (end 83.59 37.09) (width 0.2) (layer "F.Cu") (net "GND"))
 (segment (start 32.175 41.405) (end 41.522 41.405) (width 0.2) (layer "F.Cu") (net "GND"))
 (segment (start 49.5365 33.4565) (end 52.2035 36.1235) (width 0.2) (layer "F.Cu") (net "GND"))
 (segment (start 65.0535 36.1235) (end 67.7435 33.4335) (width 0.2) (layer "F.Cu") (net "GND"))
 (segment (start 70.9235 33.4335) (end 67.7435 33.4335) (width 0.2) (layer "F.Cu") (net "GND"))
 (segment (start 75.5 48.949999) (end 76.350001 49.8) (width 0.2) (layer "F.Cu") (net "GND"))
 (segment (start 83.59 37.09) (end 83.59 44.959943) (width 0.2) (layer "F.Cu") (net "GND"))
 (segment (start 75.2885 37.7985) (end 70.9235 33.4335) (width 0.2) (layer "F.Cu") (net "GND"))
 (via (at 78.5 33) (size 0.6) (drill 0.3) (layers "F.Cu" "B.Cu") (capping no) (covering (front no) (back no))
  (plugging (front no) (back no)) (filling no) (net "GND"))
 (via (at 75.438008 39.25) (size 0.6) (drill 0.3) (layers "F.Cu" "B.Cu") (capping no) (covering (front no) (back no))
  (plugging (front no) (back no)) (filling no) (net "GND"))
 (segment (start 78.5 34.3) (end 78.5 33) (width 0.2) (layer "B.Cu") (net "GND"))
 (segment (start 78.3 39.25) (end 75.438008 39.25) (width 0.2) (layer "B.Cu") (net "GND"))
 (segment (start 83.01 41.75) (end 80.8 41.75) (width 0.2) (layer "B.Cu") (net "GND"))
 (segment (start 75.438008 39.25) (end 75.438008 37.361992) (width 0.2) (layer "B.Cu") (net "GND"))
 (segment (start 83.9 40.86) (end 83.01 41.75) (width 0.2) (layer "B.Cu") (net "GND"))
 (segment (start 75.438008 37.361992) (end 78.5 34.3) (width 0.2) (layer "B.Cu") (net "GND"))
 (segment (start 80.8 41.75) (end 78.3 39.25) (width 0.2) (layer "B.Cu") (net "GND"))
 (segment (start 36.8035 48.6635) (end 39.1835 51.0435) (width 0.2) (layer "F.Cu") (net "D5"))
 (segment (start 39.1875 51.0475) (end 52.6695 51.0475) (width 0.2) (layer "F.Cu") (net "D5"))
 (segment (start 79.929999 46.22) (end 81.788 44.361999) (width 0.2) (layer "F.Cu") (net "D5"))
 (segment (start 75.973064 46.22) (end 79.929999 46.22) (width 0.2) (layer "F.Cu") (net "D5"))
 (segment (start 55.0435 48.6735) (end 57.8 51.43) (width 0.2) (layer "F.Cu") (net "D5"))
 (segment (start 70.763064 51.43) (end 75.973064 46.22) (width 0.2) (layer "F.Cu") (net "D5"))
 (segment (start 57.8 51.43) (end 70.763064 51.43) (width 0.2) (layer "F.Cu") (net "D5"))
 (segment (start 81.788 44.361999) (end 81.788 43.406) (width 0.2) (layer "F.Cu") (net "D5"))
 (segment (start 52.6695 51.0475) (end 55.0435 48.6735) (width 0.2) (layer "F.Cu") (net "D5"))
 (segment (start 57.5835 48.6735) (end 59.93 51.02) (width 0.2) (layer "F.Cu") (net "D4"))
 (segment (start 52.6935 49.52019) (end 54.79019 47.4235) (width 0.2) (layer "F.Cu") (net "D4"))
 (segment (start 59.93 51.02) (end 70.445032 51.02) (width 0.2) (layer "F.Cu") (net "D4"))
 (segment (start 54.79019 47.4235) (end 56.3335 47.4235) (width 0.2) (layer "F.Cu") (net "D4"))
 (segment (start 45.8264 50.6335) (end 45.8394 50.6465) (width 0.2) (layer "F.Cu") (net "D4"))
 (segment (start 52.6935 49.5235) (end 52.6935 49.52019) (width 0.2) (layer "F.Cu") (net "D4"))
 (segment (start 70.445032 51.02) (end 75.755032 45.71) (width 0.2) (layer "F.Cu") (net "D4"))
 (segment (start 39.3435 48.6635) (end 41.3135 50.6335) (width 0.2) (layer "F.Cu") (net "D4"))
 (segment (start 45.8394 50.6465) (end 51.5705 50.6465) (width 0.2) (layer "F.Cu") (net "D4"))
 (segment (start 41.3135 50.6335) (end 45.8264 50.6335) (width 0.2) (layer "F.Cu") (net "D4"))
 (segment (start 78.095 45.71) (end 79.226 44.579) (width 0.2) (layer "F.Cu") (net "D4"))
 (segment (start 51.5705 50.6465) (end 52.6935 49.5235) (width 0.2) (layer "F.Cu") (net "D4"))
 (segment (start 79.226 44.579) (end 79.226 43.384) (width 0.2) (layer "F.Cu") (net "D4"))
 (segment (start 75.755032 45.71) (end 78.095 45.71) (width 0.2) (layer "F.Cu") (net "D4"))
 (segment (start 56.3335 47.4235) (end 57.5835 48.6735) (width 0.2) (layer "F.Cu") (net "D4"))
 (segment (start 44.7255 45.8215) (end 41.8835 48.6635) (width 0.2) (layer "F.Cu") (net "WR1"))
 (segment (start 75.3 41.15) (end 73.167 41.15) (width 0.2) (layer "F.Cu") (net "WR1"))
 (segment (start 80.518 38.732) (end 80.518 38.217) (width 0.2) (layer "F.Cu") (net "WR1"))
 (segment (start 76.4 40.100735) (end 79.149265 40.100735) (width 0.2) (layer "F.Cu") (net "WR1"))
 (segment (start 67 45.8215) (end 44.7255 45.8215) (width 0.2) (layer "F.Cu") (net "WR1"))
 (segment (start 68.4935 45.8235) (end 68.524532 45.792468) (width 0.2) (layer "F.Cu") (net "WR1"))
 (segment (start 79.149265 40.100735) (end 80.518 38.732) (width 0.2) (layer "F.Cu") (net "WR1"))
 (segment (start 73.167 41.15) (end 68.4935 45.8235) (width 0.2) (layer "F.Cu") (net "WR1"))
 (via (at 67 45.8215) (size 0.6) (drill 0.3) (layers "F.Cu" "B.Cu") (capping no) (covering (front no) (back no))
  (plugging (front no) (back no)) (filling no) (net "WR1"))
 (via (at 76.4 40.100735) (size 0.6) (drill 0.3) (layers "F.Cu" "B.Cu") (capping no) (covering (front no) (back no))
  (plugging (front no) (back no)) (filling no) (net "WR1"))
 (via (at 75.3 41.15) (size 0.6) (drill 0.3) (layers "F.Cu" "B.Cu") (capping no) (covering (front no) (back no))
  (plugging (front no) (back no)) (filling no) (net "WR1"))
 (via (at 68.4935 45.8235) (size 0.6) (drill 0.3) (layers "F.Cu" "B.Cu") (capping no) (covering (front no) (back no))
  (plugging (front no) (back no)) (filling no) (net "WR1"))
 (segment (start 66.9425 45.8465) (end 66.9405 45.8445) (width 0.2) (layer "B.Cu") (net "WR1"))
 (segment (start 76.349265 40.100735) (end 76.4 40.100735) (width 0.2) (layer "B.Cu") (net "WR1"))
 (segment (start 68.4705 45.8465) (end 66.9425 45.8465) (width 0.2) (layer "B.Cu") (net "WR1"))
 (segment (start 75.3 41.15) (end 76.349265 40.100735) (width 0.2) (layer "B.Cu") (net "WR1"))
 (segment (start 68.4935 45.8235) (end 68.4705 45.8465) (width 0.2) (layer "B.Cu") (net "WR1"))
 (segment (start 61.0135 47.0235) (end 62.6635 48.6735) (width 0.2) (layer "F.Cu") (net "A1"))
 (segment (start 46.0055 50.2455) (end 50.7715 50.2455) (width 0.2) (layer "F.Cu") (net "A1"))
 (segment (start 53.9935 47.0235) (end 61.0135 47.0235) (width 0.2) (layer "F.Cu") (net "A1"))
 (segment (start 75.215032 44.85) (end 76.355 44.85) (width 0.2) (layer "F.Cu") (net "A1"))
 (segment (start 76.686 44.519) (end 76.686 43.384) (width 0.2) (layer "F.Cu") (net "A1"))
 (segment (start 62.6635 48.6735) (end 64.16 50.17) (width 0.2) (layer "F.Cu") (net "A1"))
 (segment (start 50.7715 50.2455) (end 53.9935 47.0235) (width 0.2) (layer "F.Cu") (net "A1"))
 (segment (start 44.4235 48.6635) (end 46.0055 50.2455) (width 0.2) (layer "F.Cu") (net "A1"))
 (segment (start 69.895032 50.17) (end 75.215032 44.85) (width 0.2) (layer "F.Cu") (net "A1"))
 (segment (start 64.16 50.17) (end 69.895032 50.17) (width 0.2) (layer "F.Cu") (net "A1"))
 (segment (start 76.355 44.85) (end 76.686 44.519) (width 0.2) (layer "F.Cu") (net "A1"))
 (segment (start 50.1655 49.8215) (end 53.3635 46.6235) (width 0.2) (layer "F.Cu") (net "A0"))
 (segment (start 69.585032 49.75) (end 75.432532 43.9025) (width 0.2) (layer "F.Cu") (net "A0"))
 (segment (start 66.28 49.75) (end 69.585032 49.75) (width 0.2) (layer "F.Cu") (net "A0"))
 (segment (start 46.9635 48.6635) (end 48.1215 49.8215) (width 0.2) (layer "F.Cu") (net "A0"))
 (segment (start 63.1535 46.6235) (end 65.2035 48.6735) (width 0.2) (layer "F.Cu") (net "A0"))
 (segment (start 53.3635 46.6235) (end 63.1535 46.6235) (width 0.2) (layer "F.Cu") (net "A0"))
 (segment (start 48.1215 49.8215) (end 50.1655 49.8215) (width 0.2) (layer "F.Cu") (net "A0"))
 (segment (start 65.2035 48.6735) (end 66.28 49.75) (width 0.2) (layer "F.Cu") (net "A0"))
 (segment (start 46.9635 33.4235) (end 48.0395 32.3475) (width 0.2) (layer "F.Cu") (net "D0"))
 (segment (start 48.0395 32.3475) (end 50.1775 32.3475) (width 0.2) (layer "F.Cu") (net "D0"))
 (segment (start 67.1165 35.3465) (end 67.1465 35.3465) (width 0.2) (layer "F.Cu") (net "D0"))
 (segment (start 72.898 38.367) (end 70.167 38.367) (width 0.2) (layer "F.Cu") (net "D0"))
 (segment (start 62.8935 35.7235) (end 65.1835 33.4335) (width 0.2) (layer "F.Cu") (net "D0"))
 (segment (start 50.1775 32.3475) (end 53.5525 35.7225) (width 0.2) (layer "F.Cu") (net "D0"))
 (segment (start 67.1465 35.3465) (end 70.167 38.367) (width 0.2) (layer "F.Cu") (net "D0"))
 (segment (start 53.5535 35.7235) (end 62.8935 35.7235) (width 0.2) (layer "F.Cu") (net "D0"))
 (via (at 67.1165 35.3465) (size 0.6) (drill 0.3) (layers "F.Cu" "B.Cu") (capping no) (covering (front no) (back no))
  (plugging (front no) (back no)) (filling no) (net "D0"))
 (segment (start 67.1165 35.3465) (end 65.4505 33.6805) (width 0.2) (layer "B.Cu") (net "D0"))
 (segment (start 50.5465 31.9465) (end 53.9235 35.3235) (width 0.2) (layer "F.Cu") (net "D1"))
 (segment (start 70.325516 32.2235) (end 63.8735 32.2235) (width 0.2) (layer "F.Cu") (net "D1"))
 (segment (start 53.9235 35.3235) (end 60.7735 35.3235) (width 0.2) (layer "F.Cu") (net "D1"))
 (segment (start 76.708 38.367) (end 76.708 37.367001) (width 0.2) (layer "F.Cu") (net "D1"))
 (segment (start 74.804016 36.702) (end 70.325516 32.2235) (width 0.2) (layer "F.Cu") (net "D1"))
 (segment (start 63.8735 32.2235) (end 62.6635 33.4335) (width 0.2) (layer "F.Cu") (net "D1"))
 (segment (start 76.708 37.367001) (end 76.042999 36.702) (width 0.2) (layer "F.Cu") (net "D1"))
 (segment (start 76.042999 36.702) (end 74.804016 36.702) (width 0.2) (layer "F.Cu") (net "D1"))
 (segment (start 60.7735 35.3235) (end 62.6635 33.4335) (width 0.2) (layer "F.Cu") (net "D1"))
 (segment (start 43.9805 33.4565) (end 45.4905 31.9465) (width 0.2) (layer "F.Cu") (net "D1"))
 (segment (start 45.4905 31.9465) (end 50.5465 31.9465) (width 0.2) (layer "F.Cu") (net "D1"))
 (segment (start 74.991 36.301) (end 76.911999 36.301) (width 0.2) (layer "F.Cu") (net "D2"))
 (segment (start 50.7765 31.5465) (end 43.3505 31.5465) (width 0.2) (layer "F.Cu") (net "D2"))
 (segment (start 43.3505 31.5465) (end 41.4405 33.4565) (width 0.2) (layer "F.Cu") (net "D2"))
 (segment (start 58.6335 34.9235) (end 54.1535 34.9235) (width 0.2) (layer "F.Cu") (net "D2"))
 (segment (start 61.8335 31.7235) (end 70.0935 31.7235) (width 0.2) (layer "F.Cu") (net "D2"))
 (segment (start 76.911999 36.301) (end 77.978 37.367001) (width 0.2) (layer "F.Cu") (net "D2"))
 (segment (start 77.978 37.367001) (end 77.978 38.367) (width 0.2) (layer "F.Cu") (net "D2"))
 (segment (start 70.0935 31.7235) (end 70.4135 31.7235) (width 0.2) (layer "F.Cu") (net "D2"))
 (segment (start 70.4135 31.7235) (end 74.991 36.301) (width 0.2) (layer "F.Cu") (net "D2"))
 (segment (start 54.1535 34.9235) (end 50.7765 31.5465) (width 0.2) (layer "F.Cu") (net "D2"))
 (segment (start 60.1235 33.4335) (end 58.6335 34.9235) (width 0.2) (layer "F.Cu") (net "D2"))
 (segment (start 70.0935 31.7235) (end 70.2935 31.7235) (width 0.2) (layer "F.Cu") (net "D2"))
 (segment (start 60.1235 33.4335) (end 61.8335 31.7235) (width 0.2) (layer "F.Cu") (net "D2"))
 (segment (start 32.175 36.325) (end 36.442 36.325) (width 0.2) (layer "F.Cu") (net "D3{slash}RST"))
 (segment (start 41.6205 31.1465) (end 51.0165 31.1465) (width 0.2) (layer "F.Cu") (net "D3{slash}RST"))
 (segment (start 79.248 37.367001) (end 79.248 38.367) (width 0.2) (layer "F.Cu") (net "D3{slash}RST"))
 (segment (start 54.3935 34.5235) (end 56.4935 34.5235) (width 0.2) (layer "F.Cu") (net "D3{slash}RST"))
 (segment (start 59.7935 31.2235) (end 70.5435 31.2235) (width 0.2) (layer "F.Cu") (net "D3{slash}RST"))
 (segment (start 36.442 36.325) (end 39.3435 33.4235) (width 0.2) (layer "F.Cu") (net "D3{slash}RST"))
 (segment (start 57.5835 33.4335) (end 59.7935 31.2235) (width 0.2) (layer "F.Cu") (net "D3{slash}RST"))
 (segment (start 56.4935 34.5235) (end 57.5835 33.4335) (width 0.2) (layer "F.Cu") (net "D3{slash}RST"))
 (segment (start 39.3435 33.4235) (end 41.6205 31.1465) (width 0.2) (layer "F.Cu") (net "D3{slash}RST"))
 (segment (start 70.5435 31.2235) (end 75.22 35.9) (width 0.2) (layer "F.Cu") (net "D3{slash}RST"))
 (segment (start 51.0165 31.1465) (end 54.3935 34.5235) (width 0.2) (layer "F.Cu") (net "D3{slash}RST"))
 (segment (start 75.22 35.9) (end 77.780999 35.9) (width 0.2) (layer "F.Cu") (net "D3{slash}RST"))
 (segment (start 77.780999 35.9) (end 79.248 37.367001) (width 0.2) (layer "F.Cu") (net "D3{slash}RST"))
 (segment (start 81.788 38.143) (end 81.788 37.37675) (width 0.2) (layer "F.Cu") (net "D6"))
 (segment (start 57.7105 30.7665) (end 55.0435 33.4335) (width 0.2) (layer "F.Cu") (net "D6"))
 (segment (start 39.4815 30.7455) (end 52.3555 30.7455) (width 0.2) (layer "F.Cu") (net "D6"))
 (segment (start 36.8035 33.4235) (end 39.4815 30.7455) (width 0.2) (layer "F.Cu") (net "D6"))
 (segment (start 79.91125 35.5) (end 75.53 35.5) (width 0.2) (layer "F.Cu") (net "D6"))
 (segment (start 75.53 35.5) (end 70.7965 30.7665) (width 0.2) (layer "F.Cu") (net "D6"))
 (segment (start 70.7965 30.7665) (end 57.7105 30.7665) (width 0.2) (layer "F.Cu") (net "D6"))
 (segment (start 52.3555 30.7455) (end 55.0435 33.4335) (width 0.2) (layer "F.Cu") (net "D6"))
 (segment (start 81.788 37.37675) (end 79.91125 35.5) (width 0.2) (layer "F.Cu") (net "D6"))
 (segment (start 77.115 45.29) (end 77.956 44.449) (width 0.2) (layer "F.Cu") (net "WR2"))
 (segment (start 75.455032 45.29) (end 77.115 45.29) (width 0.2) (layer "F.Cu") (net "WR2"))
 (segment (start 60.1235 48.6735) (end 62.04 50.59) (width 0.2) (layer "F.Cu") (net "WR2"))
 (segment (start 70.155032 50.59) (end 75.455032 45.29) (width 0.2) (layer "F.Cu") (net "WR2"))
 (segment (start 77.956 44.449) (end 77.956 43.384) (width 0.2) (layer "F.Cu") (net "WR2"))
 (segment (start 62.04 50.59) (end 70.155032 50.59) (width 0.2) (layer "F.Cu") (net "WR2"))
 (segment (start 80.521 42.5) (end 80.521 43.359) (width 0.2) (layer "F.Cu") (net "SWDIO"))
 (via (at 80.521 42.5) (size 0.6) (drill 0.3) (layers "F.Cu" "B.Cu") (capping no) (covering (front no) (back no))
  (plugging (front no) (back no)) (filling no) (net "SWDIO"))
 (segment (start 83 42.5) (end 83.9 43.4) (width 0.2) (layer "B.Cu") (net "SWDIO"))
 (segment (start 80.521 42.5) (end 83 42.5) (width 0.2) (layer "B.Cu") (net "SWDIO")))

